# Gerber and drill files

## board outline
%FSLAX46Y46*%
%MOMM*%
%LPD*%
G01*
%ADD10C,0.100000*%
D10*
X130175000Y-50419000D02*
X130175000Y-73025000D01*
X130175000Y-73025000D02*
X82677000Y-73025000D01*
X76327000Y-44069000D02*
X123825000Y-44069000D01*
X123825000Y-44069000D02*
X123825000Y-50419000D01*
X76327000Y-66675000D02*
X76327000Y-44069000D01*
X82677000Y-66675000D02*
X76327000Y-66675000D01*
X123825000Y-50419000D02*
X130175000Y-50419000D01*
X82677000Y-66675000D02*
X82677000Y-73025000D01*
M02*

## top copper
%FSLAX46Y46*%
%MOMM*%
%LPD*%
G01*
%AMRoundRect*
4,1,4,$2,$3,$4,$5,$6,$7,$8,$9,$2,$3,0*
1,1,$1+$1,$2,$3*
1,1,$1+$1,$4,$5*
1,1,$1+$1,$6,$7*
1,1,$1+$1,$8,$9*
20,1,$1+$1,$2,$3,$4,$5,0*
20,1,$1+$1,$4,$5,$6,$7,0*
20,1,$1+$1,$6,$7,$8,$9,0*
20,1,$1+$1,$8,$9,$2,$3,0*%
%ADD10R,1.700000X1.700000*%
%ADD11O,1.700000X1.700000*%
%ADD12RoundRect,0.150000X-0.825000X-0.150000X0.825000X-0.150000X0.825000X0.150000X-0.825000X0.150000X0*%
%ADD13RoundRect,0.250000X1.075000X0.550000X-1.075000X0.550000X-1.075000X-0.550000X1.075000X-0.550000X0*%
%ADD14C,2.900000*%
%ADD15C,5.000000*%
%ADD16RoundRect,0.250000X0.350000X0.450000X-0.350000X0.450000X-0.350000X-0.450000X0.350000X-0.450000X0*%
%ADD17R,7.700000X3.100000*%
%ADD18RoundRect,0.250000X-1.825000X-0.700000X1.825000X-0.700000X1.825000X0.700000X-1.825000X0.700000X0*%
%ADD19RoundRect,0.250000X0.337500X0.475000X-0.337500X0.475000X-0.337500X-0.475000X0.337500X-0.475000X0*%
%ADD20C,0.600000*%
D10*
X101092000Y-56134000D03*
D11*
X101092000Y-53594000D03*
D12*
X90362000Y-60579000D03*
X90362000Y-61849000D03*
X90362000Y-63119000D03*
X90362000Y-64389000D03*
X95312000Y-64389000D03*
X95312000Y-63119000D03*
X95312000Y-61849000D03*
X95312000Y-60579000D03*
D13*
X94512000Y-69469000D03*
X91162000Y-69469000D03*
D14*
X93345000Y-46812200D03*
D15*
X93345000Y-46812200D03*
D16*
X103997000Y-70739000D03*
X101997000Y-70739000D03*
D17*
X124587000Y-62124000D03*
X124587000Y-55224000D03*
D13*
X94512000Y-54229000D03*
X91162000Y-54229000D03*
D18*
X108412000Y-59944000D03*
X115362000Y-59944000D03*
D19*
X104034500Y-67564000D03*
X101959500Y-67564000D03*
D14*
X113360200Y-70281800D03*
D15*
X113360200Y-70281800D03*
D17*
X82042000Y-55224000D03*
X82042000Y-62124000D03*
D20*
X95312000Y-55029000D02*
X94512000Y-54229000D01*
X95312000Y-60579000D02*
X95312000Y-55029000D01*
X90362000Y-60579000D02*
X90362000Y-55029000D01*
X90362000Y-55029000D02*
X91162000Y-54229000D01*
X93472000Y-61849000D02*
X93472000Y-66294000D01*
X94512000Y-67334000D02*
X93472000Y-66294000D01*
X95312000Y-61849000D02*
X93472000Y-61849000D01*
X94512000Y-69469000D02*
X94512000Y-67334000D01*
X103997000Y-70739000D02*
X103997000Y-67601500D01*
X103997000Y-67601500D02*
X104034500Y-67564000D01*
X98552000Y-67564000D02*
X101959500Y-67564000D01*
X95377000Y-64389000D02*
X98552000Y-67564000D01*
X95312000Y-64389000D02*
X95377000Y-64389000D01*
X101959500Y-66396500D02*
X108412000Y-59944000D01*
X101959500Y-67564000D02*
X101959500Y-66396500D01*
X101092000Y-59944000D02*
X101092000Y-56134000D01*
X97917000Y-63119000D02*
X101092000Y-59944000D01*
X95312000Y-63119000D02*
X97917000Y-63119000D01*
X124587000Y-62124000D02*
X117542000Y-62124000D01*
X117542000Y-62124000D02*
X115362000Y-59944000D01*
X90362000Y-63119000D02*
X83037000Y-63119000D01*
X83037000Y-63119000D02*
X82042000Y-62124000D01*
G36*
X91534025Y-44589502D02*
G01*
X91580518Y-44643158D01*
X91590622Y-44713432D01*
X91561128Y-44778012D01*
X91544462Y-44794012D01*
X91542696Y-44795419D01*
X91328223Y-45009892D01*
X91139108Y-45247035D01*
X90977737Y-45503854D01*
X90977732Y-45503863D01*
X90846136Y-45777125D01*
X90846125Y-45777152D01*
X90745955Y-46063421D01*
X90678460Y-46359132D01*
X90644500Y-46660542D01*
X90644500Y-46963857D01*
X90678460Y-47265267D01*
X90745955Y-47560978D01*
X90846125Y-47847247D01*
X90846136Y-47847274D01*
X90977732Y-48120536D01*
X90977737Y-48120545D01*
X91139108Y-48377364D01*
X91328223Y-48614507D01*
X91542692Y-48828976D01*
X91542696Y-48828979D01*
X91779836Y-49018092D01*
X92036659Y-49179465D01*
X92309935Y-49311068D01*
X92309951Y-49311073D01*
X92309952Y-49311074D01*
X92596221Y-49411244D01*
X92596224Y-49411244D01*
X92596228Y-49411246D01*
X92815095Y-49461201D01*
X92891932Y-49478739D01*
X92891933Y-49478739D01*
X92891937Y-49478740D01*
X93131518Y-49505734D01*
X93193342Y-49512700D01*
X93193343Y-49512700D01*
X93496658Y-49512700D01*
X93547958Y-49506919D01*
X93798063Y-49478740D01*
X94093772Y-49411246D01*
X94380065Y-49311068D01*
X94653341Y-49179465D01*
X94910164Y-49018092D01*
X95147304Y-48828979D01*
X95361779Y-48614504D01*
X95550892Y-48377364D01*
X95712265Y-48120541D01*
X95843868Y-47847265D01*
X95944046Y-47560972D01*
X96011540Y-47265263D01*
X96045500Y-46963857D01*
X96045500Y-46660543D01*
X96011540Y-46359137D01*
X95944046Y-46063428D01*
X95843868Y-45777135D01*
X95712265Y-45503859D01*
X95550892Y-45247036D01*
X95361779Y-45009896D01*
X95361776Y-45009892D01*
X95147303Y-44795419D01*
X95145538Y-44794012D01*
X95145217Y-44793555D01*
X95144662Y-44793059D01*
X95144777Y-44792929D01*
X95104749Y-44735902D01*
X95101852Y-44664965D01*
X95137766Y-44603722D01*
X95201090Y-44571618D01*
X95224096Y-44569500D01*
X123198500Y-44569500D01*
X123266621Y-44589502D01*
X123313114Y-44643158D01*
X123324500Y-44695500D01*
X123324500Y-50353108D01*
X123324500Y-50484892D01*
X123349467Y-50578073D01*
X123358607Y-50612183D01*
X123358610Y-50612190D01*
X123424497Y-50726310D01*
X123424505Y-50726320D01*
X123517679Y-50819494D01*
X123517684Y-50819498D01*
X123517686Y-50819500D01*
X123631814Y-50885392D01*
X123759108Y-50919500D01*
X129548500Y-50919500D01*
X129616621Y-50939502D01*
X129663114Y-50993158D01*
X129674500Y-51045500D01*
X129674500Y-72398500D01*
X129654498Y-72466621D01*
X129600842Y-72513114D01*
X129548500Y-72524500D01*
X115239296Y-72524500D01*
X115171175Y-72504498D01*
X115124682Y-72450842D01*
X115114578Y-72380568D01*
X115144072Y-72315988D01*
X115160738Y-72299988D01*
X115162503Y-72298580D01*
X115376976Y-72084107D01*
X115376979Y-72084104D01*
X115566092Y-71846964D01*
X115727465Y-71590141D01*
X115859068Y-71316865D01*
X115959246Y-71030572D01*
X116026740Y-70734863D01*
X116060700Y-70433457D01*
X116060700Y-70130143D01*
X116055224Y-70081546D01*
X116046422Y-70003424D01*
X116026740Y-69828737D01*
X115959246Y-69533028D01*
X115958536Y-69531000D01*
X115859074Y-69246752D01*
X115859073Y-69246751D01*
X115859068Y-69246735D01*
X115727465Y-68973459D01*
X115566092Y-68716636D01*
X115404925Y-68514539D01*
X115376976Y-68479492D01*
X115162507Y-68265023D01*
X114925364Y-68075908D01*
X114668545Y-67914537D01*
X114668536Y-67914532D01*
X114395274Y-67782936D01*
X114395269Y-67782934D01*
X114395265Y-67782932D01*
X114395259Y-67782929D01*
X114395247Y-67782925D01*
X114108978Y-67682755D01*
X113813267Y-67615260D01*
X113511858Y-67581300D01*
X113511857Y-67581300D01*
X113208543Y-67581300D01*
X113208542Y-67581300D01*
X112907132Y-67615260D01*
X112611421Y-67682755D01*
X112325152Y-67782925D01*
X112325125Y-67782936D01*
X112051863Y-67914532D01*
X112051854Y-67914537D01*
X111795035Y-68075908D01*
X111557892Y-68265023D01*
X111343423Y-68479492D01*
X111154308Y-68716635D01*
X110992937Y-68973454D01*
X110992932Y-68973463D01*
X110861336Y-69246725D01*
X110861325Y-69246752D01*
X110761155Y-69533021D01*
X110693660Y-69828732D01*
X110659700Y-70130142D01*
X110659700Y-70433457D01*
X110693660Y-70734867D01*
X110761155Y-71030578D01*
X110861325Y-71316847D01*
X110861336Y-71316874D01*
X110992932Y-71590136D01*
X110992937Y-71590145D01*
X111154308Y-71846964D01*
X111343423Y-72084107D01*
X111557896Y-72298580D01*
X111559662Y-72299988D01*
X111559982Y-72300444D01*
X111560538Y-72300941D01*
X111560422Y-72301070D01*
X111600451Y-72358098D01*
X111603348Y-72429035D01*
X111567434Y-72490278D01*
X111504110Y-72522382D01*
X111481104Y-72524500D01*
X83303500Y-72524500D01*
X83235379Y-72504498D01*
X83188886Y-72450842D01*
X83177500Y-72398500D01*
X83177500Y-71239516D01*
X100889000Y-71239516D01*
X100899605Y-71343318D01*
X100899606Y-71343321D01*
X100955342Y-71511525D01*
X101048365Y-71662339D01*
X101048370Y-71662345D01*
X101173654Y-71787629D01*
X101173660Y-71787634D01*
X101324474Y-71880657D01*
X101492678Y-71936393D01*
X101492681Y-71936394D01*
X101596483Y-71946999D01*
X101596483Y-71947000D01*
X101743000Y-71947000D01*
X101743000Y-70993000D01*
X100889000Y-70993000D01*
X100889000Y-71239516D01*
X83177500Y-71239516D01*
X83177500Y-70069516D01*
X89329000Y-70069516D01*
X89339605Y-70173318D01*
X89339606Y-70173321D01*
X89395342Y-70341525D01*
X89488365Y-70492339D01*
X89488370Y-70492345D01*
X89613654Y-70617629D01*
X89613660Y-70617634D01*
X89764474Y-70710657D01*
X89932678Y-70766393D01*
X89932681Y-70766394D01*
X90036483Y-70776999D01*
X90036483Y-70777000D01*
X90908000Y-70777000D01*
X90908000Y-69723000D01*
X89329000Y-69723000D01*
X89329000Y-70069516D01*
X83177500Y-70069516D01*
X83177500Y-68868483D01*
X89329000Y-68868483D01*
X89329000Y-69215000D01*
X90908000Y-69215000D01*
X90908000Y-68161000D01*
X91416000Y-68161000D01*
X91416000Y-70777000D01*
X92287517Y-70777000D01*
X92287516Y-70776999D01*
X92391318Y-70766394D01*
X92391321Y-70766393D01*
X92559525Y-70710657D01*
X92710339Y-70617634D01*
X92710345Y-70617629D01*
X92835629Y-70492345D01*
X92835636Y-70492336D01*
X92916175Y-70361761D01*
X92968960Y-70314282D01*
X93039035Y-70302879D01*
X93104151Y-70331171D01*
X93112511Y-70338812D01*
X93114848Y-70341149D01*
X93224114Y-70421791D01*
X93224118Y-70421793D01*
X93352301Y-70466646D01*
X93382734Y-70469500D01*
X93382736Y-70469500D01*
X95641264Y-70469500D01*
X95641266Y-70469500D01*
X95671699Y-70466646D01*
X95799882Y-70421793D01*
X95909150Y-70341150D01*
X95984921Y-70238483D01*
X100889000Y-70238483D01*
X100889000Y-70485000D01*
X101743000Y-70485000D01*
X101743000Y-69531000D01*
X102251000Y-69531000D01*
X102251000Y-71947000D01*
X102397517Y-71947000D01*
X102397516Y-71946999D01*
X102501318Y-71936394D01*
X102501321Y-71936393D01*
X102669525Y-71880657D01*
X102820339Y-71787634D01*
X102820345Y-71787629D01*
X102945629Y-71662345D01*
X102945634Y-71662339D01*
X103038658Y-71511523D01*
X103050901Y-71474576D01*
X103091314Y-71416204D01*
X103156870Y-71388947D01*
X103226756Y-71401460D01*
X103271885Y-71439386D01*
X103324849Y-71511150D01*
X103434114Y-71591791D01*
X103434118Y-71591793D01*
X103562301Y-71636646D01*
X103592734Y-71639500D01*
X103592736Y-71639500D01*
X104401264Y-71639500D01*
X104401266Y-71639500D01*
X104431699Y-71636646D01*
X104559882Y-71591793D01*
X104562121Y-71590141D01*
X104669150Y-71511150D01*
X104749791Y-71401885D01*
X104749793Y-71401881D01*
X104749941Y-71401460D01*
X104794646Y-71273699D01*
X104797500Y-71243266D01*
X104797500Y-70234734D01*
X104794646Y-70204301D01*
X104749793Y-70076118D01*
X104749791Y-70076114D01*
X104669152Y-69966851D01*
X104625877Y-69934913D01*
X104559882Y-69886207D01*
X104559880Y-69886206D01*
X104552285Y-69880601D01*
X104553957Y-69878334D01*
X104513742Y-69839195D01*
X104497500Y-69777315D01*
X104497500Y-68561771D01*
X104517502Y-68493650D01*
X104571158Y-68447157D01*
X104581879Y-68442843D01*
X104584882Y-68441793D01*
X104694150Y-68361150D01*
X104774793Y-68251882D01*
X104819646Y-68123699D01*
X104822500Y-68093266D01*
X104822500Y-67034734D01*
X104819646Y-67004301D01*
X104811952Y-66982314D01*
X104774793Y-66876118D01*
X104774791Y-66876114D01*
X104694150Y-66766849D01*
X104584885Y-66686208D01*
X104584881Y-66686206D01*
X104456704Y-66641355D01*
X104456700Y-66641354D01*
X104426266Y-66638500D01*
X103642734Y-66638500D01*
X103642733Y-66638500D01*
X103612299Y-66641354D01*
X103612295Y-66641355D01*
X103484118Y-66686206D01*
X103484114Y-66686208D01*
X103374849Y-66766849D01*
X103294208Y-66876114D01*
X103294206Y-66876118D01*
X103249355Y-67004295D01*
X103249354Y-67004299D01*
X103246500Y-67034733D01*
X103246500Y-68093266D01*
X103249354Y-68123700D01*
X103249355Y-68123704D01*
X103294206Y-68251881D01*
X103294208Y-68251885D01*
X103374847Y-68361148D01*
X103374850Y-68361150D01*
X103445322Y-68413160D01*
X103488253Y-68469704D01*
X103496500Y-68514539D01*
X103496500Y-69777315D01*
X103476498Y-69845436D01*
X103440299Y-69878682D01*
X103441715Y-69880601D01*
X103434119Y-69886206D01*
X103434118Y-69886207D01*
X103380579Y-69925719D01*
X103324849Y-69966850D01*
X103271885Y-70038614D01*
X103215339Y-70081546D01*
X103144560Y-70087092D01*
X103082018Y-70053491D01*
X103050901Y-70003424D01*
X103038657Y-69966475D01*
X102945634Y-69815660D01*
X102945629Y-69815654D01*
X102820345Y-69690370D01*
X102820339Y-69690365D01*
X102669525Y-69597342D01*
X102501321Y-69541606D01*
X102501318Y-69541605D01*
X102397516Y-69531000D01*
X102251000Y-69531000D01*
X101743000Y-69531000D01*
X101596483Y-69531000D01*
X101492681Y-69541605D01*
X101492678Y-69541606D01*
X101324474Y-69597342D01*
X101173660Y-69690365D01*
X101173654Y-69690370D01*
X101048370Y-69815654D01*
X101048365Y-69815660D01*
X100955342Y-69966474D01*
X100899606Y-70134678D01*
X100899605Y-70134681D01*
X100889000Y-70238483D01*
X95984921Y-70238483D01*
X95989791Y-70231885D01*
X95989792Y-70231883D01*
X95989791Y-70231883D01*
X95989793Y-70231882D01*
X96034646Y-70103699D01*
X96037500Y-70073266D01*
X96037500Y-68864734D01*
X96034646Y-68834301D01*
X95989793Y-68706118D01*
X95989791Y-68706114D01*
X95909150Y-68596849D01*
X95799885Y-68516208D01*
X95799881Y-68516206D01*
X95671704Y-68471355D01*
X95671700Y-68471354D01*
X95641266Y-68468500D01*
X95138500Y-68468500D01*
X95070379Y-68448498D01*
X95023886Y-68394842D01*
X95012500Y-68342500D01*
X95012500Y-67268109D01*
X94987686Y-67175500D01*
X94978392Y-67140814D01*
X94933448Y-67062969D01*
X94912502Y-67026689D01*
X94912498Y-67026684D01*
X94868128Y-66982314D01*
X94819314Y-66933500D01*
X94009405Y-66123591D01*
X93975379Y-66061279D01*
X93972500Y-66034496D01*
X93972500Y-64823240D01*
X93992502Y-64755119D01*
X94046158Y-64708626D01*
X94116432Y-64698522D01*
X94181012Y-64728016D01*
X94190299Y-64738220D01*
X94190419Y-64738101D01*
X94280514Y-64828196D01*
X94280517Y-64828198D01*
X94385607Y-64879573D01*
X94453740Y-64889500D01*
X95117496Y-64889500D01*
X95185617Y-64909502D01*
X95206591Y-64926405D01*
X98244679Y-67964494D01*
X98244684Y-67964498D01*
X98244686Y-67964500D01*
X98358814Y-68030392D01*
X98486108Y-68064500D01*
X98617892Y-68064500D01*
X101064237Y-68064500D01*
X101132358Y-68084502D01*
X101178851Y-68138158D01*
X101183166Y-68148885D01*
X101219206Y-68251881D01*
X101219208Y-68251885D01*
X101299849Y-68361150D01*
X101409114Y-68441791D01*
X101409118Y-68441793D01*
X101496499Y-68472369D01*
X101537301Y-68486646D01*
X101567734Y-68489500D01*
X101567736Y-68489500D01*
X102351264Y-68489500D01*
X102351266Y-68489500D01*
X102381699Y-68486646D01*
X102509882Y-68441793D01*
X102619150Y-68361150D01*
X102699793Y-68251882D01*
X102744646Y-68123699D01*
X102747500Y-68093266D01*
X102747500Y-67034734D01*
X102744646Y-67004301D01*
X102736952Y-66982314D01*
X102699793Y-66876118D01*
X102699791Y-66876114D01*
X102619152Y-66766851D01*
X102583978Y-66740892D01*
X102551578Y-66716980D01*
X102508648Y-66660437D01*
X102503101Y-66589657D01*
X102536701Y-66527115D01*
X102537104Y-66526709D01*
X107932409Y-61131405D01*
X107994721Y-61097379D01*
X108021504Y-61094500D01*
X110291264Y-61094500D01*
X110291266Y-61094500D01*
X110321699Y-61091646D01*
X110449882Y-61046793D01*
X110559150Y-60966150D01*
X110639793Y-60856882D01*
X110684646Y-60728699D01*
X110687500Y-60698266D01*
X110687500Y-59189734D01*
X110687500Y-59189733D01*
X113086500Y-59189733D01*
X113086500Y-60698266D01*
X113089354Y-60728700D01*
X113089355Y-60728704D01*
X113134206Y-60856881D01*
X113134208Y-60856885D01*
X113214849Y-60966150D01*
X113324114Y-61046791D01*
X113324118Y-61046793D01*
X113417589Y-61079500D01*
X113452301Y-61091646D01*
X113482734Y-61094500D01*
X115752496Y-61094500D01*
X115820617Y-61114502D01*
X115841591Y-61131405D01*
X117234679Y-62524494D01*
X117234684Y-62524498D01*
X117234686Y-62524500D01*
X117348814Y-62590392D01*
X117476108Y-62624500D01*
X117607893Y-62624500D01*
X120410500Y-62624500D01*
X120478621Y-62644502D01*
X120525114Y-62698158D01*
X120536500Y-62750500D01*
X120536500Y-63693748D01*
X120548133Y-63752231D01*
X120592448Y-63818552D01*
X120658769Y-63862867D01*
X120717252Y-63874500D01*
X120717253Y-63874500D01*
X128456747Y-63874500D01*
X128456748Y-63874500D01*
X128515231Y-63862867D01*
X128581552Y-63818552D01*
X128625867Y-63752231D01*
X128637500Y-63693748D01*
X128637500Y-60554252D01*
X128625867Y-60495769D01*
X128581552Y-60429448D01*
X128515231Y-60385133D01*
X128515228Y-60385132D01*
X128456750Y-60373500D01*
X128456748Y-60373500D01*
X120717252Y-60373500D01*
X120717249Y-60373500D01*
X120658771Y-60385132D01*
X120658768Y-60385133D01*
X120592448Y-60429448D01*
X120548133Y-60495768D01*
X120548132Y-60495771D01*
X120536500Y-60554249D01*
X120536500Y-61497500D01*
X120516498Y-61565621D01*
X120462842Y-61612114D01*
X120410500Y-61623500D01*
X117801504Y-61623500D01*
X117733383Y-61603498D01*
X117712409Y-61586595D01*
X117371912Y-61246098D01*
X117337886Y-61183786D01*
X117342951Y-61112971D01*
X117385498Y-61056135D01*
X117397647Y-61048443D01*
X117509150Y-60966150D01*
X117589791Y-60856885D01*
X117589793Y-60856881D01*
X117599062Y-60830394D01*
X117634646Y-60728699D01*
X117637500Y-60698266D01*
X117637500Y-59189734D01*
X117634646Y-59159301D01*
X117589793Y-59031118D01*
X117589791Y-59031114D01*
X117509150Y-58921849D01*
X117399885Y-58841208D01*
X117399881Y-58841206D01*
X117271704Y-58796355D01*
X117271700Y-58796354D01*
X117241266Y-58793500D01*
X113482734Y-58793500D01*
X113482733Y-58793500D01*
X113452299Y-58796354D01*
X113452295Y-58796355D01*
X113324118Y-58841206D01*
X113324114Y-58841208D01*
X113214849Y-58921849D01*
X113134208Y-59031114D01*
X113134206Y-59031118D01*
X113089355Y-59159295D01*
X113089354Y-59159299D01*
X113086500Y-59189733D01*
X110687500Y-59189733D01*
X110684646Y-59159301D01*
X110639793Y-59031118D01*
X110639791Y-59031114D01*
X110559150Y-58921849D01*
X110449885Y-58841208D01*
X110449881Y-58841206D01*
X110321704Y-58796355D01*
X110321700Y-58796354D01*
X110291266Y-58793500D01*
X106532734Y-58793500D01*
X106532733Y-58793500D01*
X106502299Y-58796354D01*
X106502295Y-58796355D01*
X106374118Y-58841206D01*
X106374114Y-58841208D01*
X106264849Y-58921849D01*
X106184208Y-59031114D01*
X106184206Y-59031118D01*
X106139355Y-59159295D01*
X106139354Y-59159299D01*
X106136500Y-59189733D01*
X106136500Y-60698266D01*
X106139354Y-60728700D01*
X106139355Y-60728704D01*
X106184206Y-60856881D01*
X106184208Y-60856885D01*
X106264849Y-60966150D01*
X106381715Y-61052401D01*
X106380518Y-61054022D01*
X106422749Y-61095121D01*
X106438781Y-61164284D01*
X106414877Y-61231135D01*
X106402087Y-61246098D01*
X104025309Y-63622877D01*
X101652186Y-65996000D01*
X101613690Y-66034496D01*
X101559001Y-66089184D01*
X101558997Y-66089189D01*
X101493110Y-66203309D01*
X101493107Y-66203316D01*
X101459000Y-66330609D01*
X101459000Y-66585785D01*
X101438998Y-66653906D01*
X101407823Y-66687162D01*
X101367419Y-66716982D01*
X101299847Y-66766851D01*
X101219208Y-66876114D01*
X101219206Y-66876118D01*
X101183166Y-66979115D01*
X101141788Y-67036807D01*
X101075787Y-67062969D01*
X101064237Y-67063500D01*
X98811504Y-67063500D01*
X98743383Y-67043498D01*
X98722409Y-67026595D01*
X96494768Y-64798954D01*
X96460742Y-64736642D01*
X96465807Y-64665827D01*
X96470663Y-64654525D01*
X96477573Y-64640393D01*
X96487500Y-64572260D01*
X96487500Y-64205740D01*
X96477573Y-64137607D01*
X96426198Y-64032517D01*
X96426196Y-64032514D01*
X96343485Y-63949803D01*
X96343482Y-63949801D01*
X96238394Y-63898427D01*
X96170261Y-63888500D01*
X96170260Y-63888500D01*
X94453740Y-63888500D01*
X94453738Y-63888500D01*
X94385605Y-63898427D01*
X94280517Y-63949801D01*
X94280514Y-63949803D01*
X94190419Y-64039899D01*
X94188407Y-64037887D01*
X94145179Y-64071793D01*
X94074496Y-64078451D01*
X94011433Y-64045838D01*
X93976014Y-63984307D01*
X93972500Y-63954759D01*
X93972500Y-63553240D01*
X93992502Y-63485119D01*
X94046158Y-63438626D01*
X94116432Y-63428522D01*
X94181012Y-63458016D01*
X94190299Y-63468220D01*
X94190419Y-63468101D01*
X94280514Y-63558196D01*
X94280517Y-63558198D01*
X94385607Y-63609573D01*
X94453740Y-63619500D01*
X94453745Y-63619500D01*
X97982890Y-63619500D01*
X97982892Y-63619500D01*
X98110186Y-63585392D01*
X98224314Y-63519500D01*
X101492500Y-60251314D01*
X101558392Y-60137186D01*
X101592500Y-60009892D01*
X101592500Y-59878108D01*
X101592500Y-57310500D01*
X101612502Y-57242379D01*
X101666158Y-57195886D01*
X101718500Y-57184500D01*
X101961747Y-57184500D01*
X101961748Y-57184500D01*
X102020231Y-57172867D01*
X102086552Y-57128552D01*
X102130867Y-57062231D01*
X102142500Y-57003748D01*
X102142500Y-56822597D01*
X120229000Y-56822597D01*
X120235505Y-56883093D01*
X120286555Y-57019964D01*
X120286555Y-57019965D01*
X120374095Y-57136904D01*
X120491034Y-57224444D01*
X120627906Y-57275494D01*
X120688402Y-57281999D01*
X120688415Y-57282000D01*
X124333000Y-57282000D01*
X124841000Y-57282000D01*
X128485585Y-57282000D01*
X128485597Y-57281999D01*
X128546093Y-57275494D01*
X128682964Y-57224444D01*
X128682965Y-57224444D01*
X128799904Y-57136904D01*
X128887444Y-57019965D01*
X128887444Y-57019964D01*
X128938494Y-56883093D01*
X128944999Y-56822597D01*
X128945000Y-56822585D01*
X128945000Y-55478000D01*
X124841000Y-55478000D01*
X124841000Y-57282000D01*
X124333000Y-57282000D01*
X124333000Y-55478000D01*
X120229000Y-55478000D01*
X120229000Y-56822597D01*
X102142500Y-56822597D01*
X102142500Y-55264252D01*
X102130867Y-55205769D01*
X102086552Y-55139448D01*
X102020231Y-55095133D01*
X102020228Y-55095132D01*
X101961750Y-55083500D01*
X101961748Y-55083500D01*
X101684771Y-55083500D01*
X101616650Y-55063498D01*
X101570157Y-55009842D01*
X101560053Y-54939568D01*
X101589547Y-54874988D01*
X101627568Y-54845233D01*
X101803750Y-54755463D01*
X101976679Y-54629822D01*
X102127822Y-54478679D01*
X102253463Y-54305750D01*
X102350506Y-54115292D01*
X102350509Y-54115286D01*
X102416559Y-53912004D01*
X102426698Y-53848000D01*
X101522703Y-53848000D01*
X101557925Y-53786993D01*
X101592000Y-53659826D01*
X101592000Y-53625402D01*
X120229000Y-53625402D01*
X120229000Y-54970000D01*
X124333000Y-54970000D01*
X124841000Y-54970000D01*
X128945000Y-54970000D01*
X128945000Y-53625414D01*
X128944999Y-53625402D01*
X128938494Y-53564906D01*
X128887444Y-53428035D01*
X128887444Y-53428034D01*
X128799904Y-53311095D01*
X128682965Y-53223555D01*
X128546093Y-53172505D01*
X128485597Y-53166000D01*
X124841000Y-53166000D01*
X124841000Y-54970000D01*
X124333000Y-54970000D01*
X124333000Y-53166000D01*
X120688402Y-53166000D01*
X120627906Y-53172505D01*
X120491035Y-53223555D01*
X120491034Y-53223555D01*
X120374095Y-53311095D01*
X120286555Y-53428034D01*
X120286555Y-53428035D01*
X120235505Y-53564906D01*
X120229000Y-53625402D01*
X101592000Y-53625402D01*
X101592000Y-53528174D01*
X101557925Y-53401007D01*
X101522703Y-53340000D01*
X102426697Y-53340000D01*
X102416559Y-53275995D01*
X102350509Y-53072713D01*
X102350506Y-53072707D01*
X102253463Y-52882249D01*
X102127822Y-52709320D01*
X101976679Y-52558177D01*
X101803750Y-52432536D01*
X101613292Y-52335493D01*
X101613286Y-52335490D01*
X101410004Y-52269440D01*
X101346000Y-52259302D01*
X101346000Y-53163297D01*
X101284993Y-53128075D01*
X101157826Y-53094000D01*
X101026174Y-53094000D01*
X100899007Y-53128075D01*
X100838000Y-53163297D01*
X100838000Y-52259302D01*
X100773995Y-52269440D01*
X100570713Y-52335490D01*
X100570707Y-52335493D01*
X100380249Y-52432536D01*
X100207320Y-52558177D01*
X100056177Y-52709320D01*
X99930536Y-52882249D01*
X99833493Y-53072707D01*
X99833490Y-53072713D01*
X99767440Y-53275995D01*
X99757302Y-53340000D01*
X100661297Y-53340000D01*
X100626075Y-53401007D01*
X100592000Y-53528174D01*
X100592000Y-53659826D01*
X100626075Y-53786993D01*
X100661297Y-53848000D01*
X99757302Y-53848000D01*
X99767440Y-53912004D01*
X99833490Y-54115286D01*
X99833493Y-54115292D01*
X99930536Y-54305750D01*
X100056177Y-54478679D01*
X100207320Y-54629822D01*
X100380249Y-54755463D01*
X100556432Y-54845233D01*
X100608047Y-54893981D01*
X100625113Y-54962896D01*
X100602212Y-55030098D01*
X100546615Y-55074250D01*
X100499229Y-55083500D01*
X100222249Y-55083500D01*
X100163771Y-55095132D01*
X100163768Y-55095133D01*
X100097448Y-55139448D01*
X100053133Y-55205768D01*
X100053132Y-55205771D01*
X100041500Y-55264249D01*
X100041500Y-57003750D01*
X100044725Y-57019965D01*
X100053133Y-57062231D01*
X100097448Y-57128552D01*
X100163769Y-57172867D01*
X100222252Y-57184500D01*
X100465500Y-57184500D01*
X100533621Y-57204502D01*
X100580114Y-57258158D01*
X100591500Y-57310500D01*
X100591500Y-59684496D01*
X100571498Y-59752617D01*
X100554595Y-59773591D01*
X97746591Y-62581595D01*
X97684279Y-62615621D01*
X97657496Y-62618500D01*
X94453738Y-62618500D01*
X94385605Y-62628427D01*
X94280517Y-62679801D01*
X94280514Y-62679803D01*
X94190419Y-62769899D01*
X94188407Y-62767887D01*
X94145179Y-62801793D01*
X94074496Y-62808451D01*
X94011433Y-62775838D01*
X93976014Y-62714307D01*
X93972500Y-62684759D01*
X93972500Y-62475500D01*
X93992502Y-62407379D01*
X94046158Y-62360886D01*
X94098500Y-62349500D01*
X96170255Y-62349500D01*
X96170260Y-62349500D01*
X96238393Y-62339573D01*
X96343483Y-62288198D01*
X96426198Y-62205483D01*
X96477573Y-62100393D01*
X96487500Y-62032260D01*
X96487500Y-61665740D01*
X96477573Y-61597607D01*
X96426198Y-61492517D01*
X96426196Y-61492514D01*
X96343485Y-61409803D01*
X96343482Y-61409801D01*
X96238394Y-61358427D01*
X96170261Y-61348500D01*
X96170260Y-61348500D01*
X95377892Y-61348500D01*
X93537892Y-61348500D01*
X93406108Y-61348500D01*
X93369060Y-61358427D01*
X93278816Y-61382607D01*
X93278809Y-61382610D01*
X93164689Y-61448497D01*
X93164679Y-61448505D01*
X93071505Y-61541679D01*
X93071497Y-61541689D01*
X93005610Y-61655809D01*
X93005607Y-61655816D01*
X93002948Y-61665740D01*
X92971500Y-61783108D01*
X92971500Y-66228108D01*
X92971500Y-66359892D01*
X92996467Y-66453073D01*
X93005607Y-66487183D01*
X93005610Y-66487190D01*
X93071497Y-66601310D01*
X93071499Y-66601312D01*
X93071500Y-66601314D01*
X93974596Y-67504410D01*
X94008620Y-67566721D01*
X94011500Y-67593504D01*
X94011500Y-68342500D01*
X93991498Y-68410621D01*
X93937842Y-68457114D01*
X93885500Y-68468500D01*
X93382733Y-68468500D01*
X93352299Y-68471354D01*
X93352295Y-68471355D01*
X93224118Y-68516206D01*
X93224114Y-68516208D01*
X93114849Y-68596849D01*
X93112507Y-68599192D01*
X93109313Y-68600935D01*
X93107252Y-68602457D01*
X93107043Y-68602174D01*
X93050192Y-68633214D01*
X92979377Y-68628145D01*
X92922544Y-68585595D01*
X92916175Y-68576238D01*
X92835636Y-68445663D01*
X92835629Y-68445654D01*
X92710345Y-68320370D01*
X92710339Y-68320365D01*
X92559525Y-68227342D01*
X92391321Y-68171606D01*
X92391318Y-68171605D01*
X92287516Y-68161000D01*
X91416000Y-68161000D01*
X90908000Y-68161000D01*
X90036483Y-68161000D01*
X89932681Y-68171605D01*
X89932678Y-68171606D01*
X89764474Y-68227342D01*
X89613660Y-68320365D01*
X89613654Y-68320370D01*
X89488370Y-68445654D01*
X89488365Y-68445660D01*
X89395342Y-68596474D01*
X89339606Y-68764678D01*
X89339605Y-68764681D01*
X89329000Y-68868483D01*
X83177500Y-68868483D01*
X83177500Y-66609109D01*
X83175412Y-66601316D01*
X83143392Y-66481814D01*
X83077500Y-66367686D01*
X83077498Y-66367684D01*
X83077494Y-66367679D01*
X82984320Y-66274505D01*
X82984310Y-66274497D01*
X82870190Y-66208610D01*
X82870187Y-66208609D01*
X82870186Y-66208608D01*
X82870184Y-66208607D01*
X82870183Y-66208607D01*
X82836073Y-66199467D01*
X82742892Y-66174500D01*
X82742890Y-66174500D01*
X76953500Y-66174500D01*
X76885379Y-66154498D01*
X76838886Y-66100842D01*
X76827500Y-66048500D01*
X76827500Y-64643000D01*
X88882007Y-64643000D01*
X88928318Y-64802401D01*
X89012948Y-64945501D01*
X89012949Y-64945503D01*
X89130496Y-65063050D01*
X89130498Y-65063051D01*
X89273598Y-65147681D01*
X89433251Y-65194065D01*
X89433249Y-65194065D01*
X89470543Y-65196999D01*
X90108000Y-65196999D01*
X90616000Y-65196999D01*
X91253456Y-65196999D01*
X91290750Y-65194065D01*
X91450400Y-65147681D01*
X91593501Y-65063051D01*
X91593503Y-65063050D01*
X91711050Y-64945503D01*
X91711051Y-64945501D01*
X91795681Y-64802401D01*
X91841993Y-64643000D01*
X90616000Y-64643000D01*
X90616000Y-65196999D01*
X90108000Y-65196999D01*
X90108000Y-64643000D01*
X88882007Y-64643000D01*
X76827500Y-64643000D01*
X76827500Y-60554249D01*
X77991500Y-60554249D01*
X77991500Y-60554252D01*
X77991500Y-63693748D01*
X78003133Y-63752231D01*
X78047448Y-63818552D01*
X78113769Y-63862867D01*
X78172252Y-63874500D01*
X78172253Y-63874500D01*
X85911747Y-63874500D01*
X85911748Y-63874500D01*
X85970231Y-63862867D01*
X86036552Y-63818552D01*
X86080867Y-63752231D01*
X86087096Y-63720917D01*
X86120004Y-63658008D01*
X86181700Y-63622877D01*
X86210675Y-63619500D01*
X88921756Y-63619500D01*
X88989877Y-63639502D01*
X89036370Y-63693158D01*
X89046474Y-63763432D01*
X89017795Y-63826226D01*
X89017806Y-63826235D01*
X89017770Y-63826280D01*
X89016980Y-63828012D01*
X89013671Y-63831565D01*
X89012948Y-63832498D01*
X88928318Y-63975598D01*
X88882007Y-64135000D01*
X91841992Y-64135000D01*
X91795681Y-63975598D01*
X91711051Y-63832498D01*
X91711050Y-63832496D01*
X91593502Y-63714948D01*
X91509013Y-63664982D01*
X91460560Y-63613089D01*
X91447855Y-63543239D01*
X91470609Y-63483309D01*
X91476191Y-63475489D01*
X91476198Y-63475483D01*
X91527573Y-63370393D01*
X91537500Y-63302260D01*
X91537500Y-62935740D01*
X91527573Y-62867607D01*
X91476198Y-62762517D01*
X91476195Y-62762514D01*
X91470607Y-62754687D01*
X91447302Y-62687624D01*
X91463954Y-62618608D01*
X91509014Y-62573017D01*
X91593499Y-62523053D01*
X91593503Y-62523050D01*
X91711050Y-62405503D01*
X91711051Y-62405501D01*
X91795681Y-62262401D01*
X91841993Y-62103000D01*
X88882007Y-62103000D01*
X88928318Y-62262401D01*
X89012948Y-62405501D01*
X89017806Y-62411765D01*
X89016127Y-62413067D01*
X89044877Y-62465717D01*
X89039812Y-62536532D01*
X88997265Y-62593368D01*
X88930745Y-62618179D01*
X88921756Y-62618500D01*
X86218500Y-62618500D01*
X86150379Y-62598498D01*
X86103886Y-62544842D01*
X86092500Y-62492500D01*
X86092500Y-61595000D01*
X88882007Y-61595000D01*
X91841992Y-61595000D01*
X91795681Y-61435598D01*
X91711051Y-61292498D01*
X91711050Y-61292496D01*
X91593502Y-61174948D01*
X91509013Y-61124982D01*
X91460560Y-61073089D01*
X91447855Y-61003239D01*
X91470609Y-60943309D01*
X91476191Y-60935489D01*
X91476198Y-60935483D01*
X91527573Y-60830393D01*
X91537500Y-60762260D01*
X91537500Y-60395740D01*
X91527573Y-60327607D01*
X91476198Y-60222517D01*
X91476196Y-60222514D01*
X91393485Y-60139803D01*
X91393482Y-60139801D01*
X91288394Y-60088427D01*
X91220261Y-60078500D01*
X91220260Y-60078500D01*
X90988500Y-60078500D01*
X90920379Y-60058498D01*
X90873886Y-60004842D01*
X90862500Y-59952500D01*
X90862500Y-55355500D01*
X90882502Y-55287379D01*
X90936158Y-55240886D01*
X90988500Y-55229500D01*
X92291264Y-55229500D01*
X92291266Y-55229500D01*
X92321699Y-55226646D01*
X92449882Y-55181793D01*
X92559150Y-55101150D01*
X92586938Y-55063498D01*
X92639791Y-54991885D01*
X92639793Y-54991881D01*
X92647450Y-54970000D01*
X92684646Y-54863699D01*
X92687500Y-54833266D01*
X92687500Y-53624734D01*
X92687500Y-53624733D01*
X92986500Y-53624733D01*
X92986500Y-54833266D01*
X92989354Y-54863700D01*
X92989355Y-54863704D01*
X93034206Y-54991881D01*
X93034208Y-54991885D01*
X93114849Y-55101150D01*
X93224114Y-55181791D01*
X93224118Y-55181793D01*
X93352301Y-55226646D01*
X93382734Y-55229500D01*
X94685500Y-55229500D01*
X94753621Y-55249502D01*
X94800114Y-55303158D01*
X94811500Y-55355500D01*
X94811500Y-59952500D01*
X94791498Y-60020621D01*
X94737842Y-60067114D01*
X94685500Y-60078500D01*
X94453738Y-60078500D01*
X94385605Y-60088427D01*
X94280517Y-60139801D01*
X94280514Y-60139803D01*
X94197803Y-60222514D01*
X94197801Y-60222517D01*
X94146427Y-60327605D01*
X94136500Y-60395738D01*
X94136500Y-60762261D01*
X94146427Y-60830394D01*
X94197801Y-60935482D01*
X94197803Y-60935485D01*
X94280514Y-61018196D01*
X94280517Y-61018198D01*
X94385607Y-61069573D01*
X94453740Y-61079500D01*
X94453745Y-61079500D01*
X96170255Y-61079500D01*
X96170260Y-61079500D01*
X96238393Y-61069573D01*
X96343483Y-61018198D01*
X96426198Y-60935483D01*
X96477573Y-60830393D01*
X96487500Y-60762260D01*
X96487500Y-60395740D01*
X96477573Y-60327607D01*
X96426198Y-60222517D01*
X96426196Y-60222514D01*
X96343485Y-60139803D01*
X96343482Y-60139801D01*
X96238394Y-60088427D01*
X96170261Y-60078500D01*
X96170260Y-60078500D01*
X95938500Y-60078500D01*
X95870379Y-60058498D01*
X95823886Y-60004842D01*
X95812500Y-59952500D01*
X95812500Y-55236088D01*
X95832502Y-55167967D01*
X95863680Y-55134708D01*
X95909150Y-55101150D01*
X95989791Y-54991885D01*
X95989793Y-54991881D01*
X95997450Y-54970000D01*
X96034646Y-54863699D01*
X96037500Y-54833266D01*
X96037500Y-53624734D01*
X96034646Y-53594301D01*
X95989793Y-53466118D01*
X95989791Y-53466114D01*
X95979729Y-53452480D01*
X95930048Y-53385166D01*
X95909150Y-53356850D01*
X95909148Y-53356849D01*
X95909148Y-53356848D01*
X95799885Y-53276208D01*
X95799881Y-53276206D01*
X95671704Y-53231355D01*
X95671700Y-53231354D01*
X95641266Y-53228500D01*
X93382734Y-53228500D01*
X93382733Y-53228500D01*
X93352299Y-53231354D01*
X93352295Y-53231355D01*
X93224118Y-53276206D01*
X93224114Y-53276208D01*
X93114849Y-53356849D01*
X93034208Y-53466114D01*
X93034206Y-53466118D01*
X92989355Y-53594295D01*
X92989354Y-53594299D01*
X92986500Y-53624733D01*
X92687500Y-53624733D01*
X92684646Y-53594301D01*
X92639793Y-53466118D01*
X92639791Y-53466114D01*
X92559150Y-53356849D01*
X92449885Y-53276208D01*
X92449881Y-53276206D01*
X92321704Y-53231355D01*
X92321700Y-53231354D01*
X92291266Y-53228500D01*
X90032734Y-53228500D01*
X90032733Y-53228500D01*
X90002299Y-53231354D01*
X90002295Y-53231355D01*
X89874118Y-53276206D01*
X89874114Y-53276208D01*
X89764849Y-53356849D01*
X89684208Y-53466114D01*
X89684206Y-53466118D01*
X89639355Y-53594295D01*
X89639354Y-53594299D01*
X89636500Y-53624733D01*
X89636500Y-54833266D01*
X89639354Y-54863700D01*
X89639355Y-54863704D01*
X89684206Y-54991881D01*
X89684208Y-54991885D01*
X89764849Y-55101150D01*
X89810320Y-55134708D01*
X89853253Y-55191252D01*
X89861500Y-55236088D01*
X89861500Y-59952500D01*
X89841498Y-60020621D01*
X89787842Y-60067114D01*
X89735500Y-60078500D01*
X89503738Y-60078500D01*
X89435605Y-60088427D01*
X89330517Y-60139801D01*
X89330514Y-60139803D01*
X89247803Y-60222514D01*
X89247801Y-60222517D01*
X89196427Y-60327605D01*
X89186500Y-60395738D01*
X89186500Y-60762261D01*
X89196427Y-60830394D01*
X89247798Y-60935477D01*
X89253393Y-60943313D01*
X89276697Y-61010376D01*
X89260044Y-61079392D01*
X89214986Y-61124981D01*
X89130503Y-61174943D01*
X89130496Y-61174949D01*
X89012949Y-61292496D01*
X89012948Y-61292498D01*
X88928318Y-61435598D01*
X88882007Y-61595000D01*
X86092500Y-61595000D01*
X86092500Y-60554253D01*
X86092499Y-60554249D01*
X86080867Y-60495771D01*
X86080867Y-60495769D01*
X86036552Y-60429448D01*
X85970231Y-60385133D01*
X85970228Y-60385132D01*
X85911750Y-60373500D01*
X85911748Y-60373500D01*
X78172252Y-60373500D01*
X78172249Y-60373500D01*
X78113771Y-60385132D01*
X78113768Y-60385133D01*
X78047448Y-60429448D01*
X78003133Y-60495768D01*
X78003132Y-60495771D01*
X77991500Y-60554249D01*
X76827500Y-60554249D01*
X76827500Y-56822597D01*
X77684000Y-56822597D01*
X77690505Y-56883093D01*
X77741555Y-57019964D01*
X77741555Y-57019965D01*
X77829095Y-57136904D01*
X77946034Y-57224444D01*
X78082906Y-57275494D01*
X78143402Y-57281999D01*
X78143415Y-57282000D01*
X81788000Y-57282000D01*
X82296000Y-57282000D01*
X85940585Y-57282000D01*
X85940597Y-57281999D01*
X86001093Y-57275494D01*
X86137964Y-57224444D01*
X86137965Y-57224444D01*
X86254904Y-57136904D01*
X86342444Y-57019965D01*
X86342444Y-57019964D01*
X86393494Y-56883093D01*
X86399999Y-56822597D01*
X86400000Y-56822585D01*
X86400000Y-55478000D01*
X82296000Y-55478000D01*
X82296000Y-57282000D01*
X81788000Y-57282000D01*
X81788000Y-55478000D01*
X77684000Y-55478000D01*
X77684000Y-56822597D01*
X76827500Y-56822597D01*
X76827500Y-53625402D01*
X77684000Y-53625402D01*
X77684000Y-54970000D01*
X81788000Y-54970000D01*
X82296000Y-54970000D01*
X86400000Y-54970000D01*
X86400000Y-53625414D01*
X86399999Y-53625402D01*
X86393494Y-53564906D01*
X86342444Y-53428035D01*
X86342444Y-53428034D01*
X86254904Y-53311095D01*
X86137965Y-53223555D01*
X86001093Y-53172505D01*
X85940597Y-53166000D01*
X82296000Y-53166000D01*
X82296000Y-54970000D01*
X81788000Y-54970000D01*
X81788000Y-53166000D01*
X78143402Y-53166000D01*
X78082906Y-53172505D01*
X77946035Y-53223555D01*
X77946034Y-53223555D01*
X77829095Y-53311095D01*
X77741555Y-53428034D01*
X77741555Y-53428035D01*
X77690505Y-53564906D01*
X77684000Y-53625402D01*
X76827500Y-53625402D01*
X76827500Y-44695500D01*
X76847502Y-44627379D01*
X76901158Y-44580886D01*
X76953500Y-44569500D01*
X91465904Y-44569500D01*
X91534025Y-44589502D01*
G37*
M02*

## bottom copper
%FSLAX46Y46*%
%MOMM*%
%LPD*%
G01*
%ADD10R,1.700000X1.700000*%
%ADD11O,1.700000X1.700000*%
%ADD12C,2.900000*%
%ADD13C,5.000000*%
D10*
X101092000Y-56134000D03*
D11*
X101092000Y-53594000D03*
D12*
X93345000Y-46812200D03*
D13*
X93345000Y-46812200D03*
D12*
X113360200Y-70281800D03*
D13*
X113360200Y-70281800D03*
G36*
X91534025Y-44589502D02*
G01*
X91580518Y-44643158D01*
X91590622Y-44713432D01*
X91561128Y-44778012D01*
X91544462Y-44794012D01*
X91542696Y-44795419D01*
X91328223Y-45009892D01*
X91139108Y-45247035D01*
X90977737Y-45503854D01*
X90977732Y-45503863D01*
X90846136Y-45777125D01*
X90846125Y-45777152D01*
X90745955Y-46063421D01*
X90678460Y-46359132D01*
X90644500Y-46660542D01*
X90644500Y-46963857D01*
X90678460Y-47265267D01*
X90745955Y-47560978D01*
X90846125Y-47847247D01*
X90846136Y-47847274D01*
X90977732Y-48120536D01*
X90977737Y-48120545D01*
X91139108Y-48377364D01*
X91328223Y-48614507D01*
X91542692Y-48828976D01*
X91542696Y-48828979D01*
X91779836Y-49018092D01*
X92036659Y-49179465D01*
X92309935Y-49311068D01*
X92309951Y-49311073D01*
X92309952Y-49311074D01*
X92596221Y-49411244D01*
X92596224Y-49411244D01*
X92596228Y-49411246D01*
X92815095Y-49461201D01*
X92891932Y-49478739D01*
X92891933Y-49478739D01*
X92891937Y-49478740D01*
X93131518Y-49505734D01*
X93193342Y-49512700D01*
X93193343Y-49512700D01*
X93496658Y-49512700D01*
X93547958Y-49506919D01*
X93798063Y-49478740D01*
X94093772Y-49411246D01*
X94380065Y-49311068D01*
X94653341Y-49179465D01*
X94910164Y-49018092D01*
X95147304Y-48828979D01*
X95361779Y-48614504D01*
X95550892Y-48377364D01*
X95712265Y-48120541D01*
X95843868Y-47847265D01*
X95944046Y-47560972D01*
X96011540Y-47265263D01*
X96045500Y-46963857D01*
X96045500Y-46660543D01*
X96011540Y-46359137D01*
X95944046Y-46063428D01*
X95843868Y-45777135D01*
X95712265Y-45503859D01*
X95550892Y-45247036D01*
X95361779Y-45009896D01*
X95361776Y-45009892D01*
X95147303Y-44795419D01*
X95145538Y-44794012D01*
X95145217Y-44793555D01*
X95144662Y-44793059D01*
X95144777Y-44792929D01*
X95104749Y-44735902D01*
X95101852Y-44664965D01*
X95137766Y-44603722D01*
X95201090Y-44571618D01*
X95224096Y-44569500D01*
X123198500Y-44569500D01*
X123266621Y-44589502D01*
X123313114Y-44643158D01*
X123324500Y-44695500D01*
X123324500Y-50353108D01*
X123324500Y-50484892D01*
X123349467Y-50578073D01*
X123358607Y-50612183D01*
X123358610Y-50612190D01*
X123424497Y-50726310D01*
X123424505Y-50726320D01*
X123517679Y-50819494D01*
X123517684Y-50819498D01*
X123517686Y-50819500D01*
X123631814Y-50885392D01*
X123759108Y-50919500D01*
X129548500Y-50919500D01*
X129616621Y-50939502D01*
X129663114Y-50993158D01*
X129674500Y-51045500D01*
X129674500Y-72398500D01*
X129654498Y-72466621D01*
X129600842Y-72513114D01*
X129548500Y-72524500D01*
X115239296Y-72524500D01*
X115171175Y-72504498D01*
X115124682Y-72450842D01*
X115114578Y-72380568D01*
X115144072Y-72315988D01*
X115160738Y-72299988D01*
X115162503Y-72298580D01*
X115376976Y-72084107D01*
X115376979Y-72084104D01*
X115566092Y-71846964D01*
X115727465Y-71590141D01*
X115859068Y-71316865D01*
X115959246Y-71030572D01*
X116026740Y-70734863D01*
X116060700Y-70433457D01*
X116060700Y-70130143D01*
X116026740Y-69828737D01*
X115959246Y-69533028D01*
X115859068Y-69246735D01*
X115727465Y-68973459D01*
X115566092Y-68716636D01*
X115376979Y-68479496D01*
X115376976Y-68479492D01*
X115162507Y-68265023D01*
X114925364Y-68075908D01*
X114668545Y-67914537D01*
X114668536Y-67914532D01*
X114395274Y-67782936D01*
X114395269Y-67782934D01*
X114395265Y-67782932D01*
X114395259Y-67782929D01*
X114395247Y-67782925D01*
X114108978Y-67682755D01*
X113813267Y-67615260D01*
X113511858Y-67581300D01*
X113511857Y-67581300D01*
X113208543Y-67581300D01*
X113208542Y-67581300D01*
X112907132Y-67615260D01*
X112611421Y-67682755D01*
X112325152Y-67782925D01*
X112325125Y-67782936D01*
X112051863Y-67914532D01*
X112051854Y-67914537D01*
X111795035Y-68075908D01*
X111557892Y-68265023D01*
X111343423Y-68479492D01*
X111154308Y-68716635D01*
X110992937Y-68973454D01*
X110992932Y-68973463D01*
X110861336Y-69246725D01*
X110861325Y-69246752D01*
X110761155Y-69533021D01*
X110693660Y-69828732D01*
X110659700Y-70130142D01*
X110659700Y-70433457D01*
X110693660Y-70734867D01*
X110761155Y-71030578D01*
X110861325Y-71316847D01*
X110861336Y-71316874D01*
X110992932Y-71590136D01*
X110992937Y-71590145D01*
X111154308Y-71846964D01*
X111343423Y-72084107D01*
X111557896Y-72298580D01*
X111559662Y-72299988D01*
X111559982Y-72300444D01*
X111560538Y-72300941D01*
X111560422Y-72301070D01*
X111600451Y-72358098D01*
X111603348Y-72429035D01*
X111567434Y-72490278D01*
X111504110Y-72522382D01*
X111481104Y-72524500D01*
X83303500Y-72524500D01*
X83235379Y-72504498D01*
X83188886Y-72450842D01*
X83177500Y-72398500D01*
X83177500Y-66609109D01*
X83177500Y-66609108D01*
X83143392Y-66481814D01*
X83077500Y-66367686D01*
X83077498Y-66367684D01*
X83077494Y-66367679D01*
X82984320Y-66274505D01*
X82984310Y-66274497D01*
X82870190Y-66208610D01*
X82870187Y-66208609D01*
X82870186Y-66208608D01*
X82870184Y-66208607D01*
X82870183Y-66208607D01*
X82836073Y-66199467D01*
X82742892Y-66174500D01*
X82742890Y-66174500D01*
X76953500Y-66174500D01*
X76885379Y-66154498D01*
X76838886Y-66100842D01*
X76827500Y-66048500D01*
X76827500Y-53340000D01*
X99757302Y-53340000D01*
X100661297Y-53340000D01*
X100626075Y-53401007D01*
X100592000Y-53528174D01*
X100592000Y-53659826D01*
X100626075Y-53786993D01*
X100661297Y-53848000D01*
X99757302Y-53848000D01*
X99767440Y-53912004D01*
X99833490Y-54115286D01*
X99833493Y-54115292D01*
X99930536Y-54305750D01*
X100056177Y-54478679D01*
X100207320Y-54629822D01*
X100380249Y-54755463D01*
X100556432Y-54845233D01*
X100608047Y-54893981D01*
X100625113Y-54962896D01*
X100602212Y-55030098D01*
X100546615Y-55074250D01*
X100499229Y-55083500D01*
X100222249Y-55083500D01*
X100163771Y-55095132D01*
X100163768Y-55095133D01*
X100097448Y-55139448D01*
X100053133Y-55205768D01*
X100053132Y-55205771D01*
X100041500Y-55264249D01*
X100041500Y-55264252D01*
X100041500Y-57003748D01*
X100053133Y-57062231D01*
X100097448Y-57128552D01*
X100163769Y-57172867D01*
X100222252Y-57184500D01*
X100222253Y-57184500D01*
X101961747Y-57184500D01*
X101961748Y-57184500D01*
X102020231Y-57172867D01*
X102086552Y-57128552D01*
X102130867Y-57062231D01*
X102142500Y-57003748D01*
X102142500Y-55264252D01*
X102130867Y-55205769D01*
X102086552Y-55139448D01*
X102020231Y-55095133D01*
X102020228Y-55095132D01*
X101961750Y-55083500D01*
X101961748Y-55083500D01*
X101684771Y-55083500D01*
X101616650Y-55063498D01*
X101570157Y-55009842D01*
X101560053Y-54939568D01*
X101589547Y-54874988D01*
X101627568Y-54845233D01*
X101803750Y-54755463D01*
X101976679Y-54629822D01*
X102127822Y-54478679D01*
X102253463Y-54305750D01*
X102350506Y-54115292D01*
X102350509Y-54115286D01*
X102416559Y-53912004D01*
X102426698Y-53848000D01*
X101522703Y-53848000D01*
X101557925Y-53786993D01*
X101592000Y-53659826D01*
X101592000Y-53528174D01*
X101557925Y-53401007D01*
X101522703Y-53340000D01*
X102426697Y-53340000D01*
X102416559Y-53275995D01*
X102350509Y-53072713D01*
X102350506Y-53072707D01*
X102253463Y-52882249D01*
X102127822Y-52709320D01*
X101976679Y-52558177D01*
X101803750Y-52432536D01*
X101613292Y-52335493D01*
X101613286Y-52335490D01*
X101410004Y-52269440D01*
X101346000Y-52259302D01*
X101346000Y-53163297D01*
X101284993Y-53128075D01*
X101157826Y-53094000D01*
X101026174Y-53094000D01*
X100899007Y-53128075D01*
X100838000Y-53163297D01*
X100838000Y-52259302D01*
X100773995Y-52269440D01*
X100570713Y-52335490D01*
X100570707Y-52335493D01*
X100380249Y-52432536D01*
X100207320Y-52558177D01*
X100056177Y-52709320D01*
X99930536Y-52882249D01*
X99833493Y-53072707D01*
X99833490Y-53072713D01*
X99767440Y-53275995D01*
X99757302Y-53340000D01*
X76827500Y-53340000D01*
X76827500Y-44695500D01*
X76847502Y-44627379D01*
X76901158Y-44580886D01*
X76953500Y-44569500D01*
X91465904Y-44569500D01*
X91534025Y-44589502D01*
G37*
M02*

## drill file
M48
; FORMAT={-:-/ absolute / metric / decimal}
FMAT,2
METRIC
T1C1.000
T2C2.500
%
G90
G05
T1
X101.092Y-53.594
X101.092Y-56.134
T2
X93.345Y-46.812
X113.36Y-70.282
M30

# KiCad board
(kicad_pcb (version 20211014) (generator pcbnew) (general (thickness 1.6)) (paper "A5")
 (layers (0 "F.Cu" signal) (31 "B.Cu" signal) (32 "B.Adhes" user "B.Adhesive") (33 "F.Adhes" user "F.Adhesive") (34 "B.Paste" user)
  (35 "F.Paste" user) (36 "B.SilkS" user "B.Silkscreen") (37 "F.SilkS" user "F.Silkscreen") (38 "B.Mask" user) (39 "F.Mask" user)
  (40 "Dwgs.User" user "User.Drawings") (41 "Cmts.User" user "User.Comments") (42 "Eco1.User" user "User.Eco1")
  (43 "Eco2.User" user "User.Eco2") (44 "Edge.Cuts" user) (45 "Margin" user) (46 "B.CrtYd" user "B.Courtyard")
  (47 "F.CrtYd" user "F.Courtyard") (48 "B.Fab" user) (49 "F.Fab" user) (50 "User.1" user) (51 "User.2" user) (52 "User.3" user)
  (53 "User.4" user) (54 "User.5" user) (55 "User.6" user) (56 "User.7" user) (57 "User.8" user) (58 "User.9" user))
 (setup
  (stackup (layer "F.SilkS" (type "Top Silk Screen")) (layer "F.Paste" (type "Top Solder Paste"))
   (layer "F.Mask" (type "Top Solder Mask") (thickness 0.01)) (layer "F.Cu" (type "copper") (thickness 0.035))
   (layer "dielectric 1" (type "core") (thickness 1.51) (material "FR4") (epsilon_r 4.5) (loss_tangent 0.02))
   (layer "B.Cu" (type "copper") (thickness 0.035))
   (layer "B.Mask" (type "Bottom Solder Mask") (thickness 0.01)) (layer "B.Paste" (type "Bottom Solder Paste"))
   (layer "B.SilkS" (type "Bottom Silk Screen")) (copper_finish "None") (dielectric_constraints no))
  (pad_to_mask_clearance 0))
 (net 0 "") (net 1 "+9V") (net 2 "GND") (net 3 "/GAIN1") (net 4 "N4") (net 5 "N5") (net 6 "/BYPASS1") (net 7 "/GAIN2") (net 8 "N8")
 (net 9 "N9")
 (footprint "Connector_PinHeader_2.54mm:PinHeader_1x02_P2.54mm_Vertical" (layer "F.Cu") (at 101.092 56.134 180)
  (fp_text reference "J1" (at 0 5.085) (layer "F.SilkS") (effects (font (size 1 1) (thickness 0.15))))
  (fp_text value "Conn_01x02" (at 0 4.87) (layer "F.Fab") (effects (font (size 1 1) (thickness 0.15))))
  (pad "1" thru_hole rect (at 0 0 180) (size 1.7 1.7) (drill 1) (layers *.Cu *.Mask) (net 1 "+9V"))
  (pad "2" thru_hole oval (at 0 2.54 180) (size 1.7 1.7) (drill 1) (layers *.Cu *.Mask) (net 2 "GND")))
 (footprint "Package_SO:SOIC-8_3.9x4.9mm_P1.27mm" (layer "F.Cu") (at 92.837 62.484)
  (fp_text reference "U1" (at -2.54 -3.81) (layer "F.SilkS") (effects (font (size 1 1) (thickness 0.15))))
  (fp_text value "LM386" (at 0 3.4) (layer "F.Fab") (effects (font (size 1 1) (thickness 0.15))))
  (pad "1" smd roundrect (at -2.475 -1.905) (size 1.95 0.6) (layers "F.Cu" "F.Paste" "F.Mask") (roundrect_rratio 0.25) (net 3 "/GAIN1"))
  (pad "2" smd roundrect (at -2.475 -0.635) (size 1.95 0.6) (layers "F.Cu" "F.Paste" "F.Mask") (roundrect_rratio 0.25) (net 2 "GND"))
  (pad "3" smd roundrect (at -2.475 0.635) (size 1.95 0.6) (layers "F.Cu" "F.Paste" "F.Mask") (roundrect_rratio 0.25) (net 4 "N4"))
  (pad "4" smd roundrect (at -2.475 1.905) (size 1.95 0.6) (layers "F.Cu" "F.Paste" "F.Mask") (roundrect_rratio 0.25) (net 2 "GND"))
  (pad "5" smd roundrect (at 2.475 1.905) (size 1.95 0.6) (layers "F.Cu" "F.Paste" "F.Mask") (roundrect_rratio 0.25) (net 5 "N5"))
  (pad "6" smd roundrect (at 2.475 0.635) (size 1.95 0.6) (layers "F.Cu" "F.Paste" "F.Mask") (roundrect_rratio 0.25) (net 1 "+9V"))
  (pad "7" smd roundrect (at 2.475 -0.635) (size 1.95 0.6) (layers "F.Cu" "F.Paste" "F.Mask") (roundrect_rratio 0.25) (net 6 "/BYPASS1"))
  (pad "8" smd roundrect (at 2.475 -1.905) (size 1.95 0.6) (layers "F.Cu" "F.Paste" "F.Mask") (roundrect_rratio 0.25) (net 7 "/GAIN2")))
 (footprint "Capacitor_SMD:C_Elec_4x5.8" (layer "F.Cu") (at 92.837 69.469 180)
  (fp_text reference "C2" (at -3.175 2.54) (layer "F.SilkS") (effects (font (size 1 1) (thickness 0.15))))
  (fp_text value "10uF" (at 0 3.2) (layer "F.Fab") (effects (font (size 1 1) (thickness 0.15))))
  (pad "1" smd roundrect (at -1.675 0 180) (size 2.65 1.6) (layers "F.Cu" "F.Paste" "F.Mask") (roundrect_rratio 0.15625) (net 6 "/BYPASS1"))
  (pad "2" smd roundrect (at 1.675 0 180) (size 2.65 1.6) (layers "F.Cu" "F.Paste" "F.Mask") (roundrect_rratio 0.15625) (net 2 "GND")))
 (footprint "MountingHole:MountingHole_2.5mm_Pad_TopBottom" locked (layer "F.Cu") (at 93.345 46.8122)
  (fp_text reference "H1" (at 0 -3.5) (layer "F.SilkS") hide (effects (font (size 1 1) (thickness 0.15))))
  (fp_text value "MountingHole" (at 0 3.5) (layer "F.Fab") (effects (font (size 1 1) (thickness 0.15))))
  (pad "1" thru_hole circle locked (at 0 0) (size 2.9 2.9) (drill 2.5) (layers *.Cu *.Mask))
  (pad "1" connect circle locked (at 0 0) (size 5 5) (layers "B.Cu" "B.Mask"))
  (pad "1" connect circle locked (at 0 0) (size 5 5) (layers "F.Cu" "F.Mask")))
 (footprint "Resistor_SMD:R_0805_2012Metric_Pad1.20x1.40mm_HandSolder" (layer "F.Cu") (at 102.997 70.739 180)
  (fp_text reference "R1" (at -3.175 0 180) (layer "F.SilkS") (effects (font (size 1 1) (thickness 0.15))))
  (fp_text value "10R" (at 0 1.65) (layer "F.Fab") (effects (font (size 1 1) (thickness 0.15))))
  (pad "1" smd roundrect (at -1 0 180) (size 1.2 1.4) (layers "F.Cu" "F.Paste" "F.Mask") (roundrect_rratio 0.2083333333) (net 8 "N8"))
  (pad "2" smd roundrect (at 1 0 180) (size 1.2 1.4) (layers "F.Cu" "F.Paste" "F.Mask") (roundrect_rratio 0.2083333333) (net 2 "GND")))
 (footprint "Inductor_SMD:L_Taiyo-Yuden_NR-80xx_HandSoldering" (layer "F.Cu") (at 124.587 58.674 90)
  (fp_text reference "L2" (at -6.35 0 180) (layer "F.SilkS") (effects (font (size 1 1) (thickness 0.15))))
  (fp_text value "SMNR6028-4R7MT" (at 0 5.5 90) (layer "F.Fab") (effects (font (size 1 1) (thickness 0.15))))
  (pad "1" smd rect (at -3.45 0 90) (size 3.1 7.7) (layers "F.Cu" "F.Paste" "F.Mask") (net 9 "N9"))
  (pad "2" smd rect (at 3.45 0 90) (size 3.1 7.7) (layers "F.Cu" "F.Paste" "F.Mask") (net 2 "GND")))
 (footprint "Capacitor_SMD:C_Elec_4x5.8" (layer "F.Cu") (at 92.837 54.229 180)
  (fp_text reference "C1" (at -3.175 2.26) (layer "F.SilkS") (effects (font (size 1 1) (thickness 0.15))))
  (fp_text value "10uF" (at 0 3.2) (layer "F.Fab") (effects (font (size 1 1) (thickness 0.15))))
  (pad "1" smd roundrect (at -1.675 0 180) (size 2.65 1.6) (layers "F.Cu" "F.Paste" "F.Mask") (roundrect_rratio 0.15625) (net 7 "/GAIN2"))
  (pad "2" smd roundrect (at 1.675 0 180) (size 2.65 1.6) (layers "F.Cu" "F.Paste" "F.Mask") (roundrect_rratio 0.15625) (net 3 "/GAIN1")))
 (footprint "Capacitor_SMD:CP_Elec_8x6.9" (layer "F.Cu") (at 111.887 59.944)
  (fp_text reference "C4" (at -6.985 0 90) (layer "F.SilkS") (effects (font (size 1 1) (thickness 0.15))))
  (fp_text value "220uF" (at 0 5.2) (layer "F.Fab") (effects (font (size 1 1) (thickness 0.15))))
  (pad "1" smd roundrect (at -3.475 0) (size 4.15 1.9) (layers "F.Cu" "F.Paste" "F.Mask") (roundrect_rratio 0.1315789474) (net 5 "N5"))
  (pad "2" smd roundrect (at 3.475 0) (size 4.15 1.9) (layers "F.Cu" "F.Paste" "F.Mask") (roundrect_rratio 0.1315789474) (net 9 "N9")))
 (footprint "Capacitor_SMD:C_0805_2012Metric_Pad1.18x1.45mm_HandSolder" (layer "F.Cu") (at 102.997 67.564 180)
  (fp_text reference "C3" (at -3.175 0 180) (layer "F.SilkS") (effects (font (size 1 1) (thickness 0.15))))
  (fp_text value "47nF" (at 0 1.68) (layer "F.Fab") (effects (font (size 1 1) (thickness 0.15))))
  (pad "1" smd roundrect (at -1.0375 0 180) (size 1.175 1.45) (layers "F.Cu" "F.Paste" "F.Mask") (roundrect_rratio 0.2127659574)
   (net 8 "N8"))
  (pad "2" smd roundrect (at 1.0375 0 180) (size 1.175 1.45) (layers "F.Cu" "F.Paste" "F.Mask") (roundrect_rratio 0.2127659574) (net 5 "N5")))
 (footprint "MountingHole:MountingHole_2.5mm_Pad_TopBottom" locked (layer "F.Cu") (at 113.3602 70.2818)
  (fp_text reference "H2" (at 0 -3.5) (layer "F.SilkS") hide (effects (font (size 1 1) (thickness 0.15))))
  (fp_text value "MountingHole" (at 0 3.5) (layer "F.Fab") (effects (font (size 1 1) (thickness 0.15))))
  (pad "1" thru_hole circle locked (at 0 0) (size 2.9 2.9) (drill 2.5) (layers *.Cu *.Mask))
  (pad "1" connect circle locked (at 0 0) (size 5 5) (layers "F.Cu" "F.Mask"))
  (pad "1" connect circle locked (at 0 0) (size 5 5) (layers "B.Cu" "B.Mask")))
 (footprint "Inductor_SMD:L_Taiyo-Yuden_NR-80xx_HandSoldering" (layer "F.Cu") (at 82.042 58.674 -90)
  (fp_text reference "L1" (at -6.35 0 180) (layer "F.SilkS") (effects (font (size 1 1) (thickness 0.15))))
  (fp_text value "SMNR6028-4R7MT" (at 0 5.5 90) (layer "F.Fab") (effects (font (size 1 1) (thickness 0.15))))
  (pad "1" smd rect (at -3.45 0 270) (size 3.1 7.7) (layers "F.Cu" "F.Paste" "F.Mask") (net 2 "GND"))
  (pad "2" smd rect (at 3.45 0 270) (size 3.1 7.7) (layers "F.Cu" "F.Paste" "F.Mask") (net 4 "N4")))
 (gr_line (start 130.175 50.419) (end 130.175 73.025) (layer "Edge.Cuts") (width 0.1))
 (gr_line (start 130.175 73.025) (end 82.677 73.025) (layer "Edge.Cuts") (width 0.1))
 (gr_line (start 76.327 44.069) (end 123.825 44.069) (layer "Edge.Cuts") (width 0.1))
 (gr_line (start 123.825 44.069) (end 123.825 50.419) (layer "Edge.Cuts") (width 0.1))
 (gr_line (start 76.327 66.675) (end 76.327 44.069) (layer "Edge.Cuts") (width 0.1))
 (gr_line (start 82.677 66.675) (end 76.327 66.675) (layer "Edge.Cuts") (width 0.1))
 (gr_line (start 123.825 50.419) (end 130.175 50.419) (layer "Edge.Cuts") (width 0.1))
 (gr_line (start 82.677 66.675) (end 82.677 73.025) (layer "Edge.Cuts") (width 0.1))
 (segment (start 95.312 55.029) (end 94.512 54.229) (width 0.6) (layer "F.Cu") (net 7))
 (segment (start 95.312 60.579) (end 95.312 55.029) (width 0.6) (layer "F.Cu") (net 7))
 (segment (start 90.362 60.579) (end 90.362 55.029) (width 0.6) (layer "F.Cu") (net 3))
 (segment (start 90.362 55.029) (end 91.162 54.229) (width 0.6) (layer "F.Cu") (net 3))
 (segment (start 93.472 61.849) (end 93.472 66.294) (width 0.6) (layer "F.Cu") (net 6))
 (segment (start 94.512 67.334) (end 93.472 66.294) (width 0.6) (layer "F.Cu") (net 6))
 (segment (start 95.312 61.849) (end 93.472 61.849) (width 0.6) (layer "F.Cu") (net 6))
 (segment (start 94.512 69.469) (end 94.512 67.334) (width 0.6) (layer "F.Cu") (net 6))
 (segment (start 103.997 70.739) (end 103.997 67.6015) (width 0.6) (layer "F.Cu") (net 8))
 (segment (start 103.997 67.6015) (end 104.0345 67.564) (width 0.6) (layer "F.Cu") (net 8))
 (segment (start 98.552 67.564) (end 101.9595 67.564) (width 0.6) (layer "F.Cu") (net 5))
 (segment (start 95.377 64.389) (end 98.552 67.564) (width 0.6) (layer "F.Cu") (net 5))
 (segment (start 95.312 64.389) (end 95.377 64.389) (width 0.6) (layer "F.Cu") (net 5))
 (segment (start 101.9595 66.3965) (end 108.412 59.944) (width 0.6) (layer "F.Cu") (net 5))
 (segment (start 101.9595 67.564) (end 101.9595 66.3965) (width 0.6) (layer "F.Cu") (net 5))
 (segment (start 101.092 59.944) (end 101.092 56.134) (width 0.6) (layer "F.Cu") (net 1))
 (segment (start 97.917 63.119) (end 101.092 59.944) (width 0.6) (layer "F.Cu") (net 1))
 (segment (start 95.312 63.119) (end 97.917 63.119) (width 0.6) (layer "F.Cu") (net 1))
 (segment (start 124.587 62.124) (end 117.542 62.124) (width 0.6) (layer "F.Cu") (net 9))
 (segment (start 117.542 62.124) (end 115.362 59.944) (width 0.6) (layer "F.Cu") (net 9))
 (segment (start 90.362 63.119) (end 83.037 63.119) (width 0.6) (layer "F.Cu") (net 4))
 (segment (start 83.037 63.119) (end 82.042 62.124) (width 0.6) (layer "F.Cu") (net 4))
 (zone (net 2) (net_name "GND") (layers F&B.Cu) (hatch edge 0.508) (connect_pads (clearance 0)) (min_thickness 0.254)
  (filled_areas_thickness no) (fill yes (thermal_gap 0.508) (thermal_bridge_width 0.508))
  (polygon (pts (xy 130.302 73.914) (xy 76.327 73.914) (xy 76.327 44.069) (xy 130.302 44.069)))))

